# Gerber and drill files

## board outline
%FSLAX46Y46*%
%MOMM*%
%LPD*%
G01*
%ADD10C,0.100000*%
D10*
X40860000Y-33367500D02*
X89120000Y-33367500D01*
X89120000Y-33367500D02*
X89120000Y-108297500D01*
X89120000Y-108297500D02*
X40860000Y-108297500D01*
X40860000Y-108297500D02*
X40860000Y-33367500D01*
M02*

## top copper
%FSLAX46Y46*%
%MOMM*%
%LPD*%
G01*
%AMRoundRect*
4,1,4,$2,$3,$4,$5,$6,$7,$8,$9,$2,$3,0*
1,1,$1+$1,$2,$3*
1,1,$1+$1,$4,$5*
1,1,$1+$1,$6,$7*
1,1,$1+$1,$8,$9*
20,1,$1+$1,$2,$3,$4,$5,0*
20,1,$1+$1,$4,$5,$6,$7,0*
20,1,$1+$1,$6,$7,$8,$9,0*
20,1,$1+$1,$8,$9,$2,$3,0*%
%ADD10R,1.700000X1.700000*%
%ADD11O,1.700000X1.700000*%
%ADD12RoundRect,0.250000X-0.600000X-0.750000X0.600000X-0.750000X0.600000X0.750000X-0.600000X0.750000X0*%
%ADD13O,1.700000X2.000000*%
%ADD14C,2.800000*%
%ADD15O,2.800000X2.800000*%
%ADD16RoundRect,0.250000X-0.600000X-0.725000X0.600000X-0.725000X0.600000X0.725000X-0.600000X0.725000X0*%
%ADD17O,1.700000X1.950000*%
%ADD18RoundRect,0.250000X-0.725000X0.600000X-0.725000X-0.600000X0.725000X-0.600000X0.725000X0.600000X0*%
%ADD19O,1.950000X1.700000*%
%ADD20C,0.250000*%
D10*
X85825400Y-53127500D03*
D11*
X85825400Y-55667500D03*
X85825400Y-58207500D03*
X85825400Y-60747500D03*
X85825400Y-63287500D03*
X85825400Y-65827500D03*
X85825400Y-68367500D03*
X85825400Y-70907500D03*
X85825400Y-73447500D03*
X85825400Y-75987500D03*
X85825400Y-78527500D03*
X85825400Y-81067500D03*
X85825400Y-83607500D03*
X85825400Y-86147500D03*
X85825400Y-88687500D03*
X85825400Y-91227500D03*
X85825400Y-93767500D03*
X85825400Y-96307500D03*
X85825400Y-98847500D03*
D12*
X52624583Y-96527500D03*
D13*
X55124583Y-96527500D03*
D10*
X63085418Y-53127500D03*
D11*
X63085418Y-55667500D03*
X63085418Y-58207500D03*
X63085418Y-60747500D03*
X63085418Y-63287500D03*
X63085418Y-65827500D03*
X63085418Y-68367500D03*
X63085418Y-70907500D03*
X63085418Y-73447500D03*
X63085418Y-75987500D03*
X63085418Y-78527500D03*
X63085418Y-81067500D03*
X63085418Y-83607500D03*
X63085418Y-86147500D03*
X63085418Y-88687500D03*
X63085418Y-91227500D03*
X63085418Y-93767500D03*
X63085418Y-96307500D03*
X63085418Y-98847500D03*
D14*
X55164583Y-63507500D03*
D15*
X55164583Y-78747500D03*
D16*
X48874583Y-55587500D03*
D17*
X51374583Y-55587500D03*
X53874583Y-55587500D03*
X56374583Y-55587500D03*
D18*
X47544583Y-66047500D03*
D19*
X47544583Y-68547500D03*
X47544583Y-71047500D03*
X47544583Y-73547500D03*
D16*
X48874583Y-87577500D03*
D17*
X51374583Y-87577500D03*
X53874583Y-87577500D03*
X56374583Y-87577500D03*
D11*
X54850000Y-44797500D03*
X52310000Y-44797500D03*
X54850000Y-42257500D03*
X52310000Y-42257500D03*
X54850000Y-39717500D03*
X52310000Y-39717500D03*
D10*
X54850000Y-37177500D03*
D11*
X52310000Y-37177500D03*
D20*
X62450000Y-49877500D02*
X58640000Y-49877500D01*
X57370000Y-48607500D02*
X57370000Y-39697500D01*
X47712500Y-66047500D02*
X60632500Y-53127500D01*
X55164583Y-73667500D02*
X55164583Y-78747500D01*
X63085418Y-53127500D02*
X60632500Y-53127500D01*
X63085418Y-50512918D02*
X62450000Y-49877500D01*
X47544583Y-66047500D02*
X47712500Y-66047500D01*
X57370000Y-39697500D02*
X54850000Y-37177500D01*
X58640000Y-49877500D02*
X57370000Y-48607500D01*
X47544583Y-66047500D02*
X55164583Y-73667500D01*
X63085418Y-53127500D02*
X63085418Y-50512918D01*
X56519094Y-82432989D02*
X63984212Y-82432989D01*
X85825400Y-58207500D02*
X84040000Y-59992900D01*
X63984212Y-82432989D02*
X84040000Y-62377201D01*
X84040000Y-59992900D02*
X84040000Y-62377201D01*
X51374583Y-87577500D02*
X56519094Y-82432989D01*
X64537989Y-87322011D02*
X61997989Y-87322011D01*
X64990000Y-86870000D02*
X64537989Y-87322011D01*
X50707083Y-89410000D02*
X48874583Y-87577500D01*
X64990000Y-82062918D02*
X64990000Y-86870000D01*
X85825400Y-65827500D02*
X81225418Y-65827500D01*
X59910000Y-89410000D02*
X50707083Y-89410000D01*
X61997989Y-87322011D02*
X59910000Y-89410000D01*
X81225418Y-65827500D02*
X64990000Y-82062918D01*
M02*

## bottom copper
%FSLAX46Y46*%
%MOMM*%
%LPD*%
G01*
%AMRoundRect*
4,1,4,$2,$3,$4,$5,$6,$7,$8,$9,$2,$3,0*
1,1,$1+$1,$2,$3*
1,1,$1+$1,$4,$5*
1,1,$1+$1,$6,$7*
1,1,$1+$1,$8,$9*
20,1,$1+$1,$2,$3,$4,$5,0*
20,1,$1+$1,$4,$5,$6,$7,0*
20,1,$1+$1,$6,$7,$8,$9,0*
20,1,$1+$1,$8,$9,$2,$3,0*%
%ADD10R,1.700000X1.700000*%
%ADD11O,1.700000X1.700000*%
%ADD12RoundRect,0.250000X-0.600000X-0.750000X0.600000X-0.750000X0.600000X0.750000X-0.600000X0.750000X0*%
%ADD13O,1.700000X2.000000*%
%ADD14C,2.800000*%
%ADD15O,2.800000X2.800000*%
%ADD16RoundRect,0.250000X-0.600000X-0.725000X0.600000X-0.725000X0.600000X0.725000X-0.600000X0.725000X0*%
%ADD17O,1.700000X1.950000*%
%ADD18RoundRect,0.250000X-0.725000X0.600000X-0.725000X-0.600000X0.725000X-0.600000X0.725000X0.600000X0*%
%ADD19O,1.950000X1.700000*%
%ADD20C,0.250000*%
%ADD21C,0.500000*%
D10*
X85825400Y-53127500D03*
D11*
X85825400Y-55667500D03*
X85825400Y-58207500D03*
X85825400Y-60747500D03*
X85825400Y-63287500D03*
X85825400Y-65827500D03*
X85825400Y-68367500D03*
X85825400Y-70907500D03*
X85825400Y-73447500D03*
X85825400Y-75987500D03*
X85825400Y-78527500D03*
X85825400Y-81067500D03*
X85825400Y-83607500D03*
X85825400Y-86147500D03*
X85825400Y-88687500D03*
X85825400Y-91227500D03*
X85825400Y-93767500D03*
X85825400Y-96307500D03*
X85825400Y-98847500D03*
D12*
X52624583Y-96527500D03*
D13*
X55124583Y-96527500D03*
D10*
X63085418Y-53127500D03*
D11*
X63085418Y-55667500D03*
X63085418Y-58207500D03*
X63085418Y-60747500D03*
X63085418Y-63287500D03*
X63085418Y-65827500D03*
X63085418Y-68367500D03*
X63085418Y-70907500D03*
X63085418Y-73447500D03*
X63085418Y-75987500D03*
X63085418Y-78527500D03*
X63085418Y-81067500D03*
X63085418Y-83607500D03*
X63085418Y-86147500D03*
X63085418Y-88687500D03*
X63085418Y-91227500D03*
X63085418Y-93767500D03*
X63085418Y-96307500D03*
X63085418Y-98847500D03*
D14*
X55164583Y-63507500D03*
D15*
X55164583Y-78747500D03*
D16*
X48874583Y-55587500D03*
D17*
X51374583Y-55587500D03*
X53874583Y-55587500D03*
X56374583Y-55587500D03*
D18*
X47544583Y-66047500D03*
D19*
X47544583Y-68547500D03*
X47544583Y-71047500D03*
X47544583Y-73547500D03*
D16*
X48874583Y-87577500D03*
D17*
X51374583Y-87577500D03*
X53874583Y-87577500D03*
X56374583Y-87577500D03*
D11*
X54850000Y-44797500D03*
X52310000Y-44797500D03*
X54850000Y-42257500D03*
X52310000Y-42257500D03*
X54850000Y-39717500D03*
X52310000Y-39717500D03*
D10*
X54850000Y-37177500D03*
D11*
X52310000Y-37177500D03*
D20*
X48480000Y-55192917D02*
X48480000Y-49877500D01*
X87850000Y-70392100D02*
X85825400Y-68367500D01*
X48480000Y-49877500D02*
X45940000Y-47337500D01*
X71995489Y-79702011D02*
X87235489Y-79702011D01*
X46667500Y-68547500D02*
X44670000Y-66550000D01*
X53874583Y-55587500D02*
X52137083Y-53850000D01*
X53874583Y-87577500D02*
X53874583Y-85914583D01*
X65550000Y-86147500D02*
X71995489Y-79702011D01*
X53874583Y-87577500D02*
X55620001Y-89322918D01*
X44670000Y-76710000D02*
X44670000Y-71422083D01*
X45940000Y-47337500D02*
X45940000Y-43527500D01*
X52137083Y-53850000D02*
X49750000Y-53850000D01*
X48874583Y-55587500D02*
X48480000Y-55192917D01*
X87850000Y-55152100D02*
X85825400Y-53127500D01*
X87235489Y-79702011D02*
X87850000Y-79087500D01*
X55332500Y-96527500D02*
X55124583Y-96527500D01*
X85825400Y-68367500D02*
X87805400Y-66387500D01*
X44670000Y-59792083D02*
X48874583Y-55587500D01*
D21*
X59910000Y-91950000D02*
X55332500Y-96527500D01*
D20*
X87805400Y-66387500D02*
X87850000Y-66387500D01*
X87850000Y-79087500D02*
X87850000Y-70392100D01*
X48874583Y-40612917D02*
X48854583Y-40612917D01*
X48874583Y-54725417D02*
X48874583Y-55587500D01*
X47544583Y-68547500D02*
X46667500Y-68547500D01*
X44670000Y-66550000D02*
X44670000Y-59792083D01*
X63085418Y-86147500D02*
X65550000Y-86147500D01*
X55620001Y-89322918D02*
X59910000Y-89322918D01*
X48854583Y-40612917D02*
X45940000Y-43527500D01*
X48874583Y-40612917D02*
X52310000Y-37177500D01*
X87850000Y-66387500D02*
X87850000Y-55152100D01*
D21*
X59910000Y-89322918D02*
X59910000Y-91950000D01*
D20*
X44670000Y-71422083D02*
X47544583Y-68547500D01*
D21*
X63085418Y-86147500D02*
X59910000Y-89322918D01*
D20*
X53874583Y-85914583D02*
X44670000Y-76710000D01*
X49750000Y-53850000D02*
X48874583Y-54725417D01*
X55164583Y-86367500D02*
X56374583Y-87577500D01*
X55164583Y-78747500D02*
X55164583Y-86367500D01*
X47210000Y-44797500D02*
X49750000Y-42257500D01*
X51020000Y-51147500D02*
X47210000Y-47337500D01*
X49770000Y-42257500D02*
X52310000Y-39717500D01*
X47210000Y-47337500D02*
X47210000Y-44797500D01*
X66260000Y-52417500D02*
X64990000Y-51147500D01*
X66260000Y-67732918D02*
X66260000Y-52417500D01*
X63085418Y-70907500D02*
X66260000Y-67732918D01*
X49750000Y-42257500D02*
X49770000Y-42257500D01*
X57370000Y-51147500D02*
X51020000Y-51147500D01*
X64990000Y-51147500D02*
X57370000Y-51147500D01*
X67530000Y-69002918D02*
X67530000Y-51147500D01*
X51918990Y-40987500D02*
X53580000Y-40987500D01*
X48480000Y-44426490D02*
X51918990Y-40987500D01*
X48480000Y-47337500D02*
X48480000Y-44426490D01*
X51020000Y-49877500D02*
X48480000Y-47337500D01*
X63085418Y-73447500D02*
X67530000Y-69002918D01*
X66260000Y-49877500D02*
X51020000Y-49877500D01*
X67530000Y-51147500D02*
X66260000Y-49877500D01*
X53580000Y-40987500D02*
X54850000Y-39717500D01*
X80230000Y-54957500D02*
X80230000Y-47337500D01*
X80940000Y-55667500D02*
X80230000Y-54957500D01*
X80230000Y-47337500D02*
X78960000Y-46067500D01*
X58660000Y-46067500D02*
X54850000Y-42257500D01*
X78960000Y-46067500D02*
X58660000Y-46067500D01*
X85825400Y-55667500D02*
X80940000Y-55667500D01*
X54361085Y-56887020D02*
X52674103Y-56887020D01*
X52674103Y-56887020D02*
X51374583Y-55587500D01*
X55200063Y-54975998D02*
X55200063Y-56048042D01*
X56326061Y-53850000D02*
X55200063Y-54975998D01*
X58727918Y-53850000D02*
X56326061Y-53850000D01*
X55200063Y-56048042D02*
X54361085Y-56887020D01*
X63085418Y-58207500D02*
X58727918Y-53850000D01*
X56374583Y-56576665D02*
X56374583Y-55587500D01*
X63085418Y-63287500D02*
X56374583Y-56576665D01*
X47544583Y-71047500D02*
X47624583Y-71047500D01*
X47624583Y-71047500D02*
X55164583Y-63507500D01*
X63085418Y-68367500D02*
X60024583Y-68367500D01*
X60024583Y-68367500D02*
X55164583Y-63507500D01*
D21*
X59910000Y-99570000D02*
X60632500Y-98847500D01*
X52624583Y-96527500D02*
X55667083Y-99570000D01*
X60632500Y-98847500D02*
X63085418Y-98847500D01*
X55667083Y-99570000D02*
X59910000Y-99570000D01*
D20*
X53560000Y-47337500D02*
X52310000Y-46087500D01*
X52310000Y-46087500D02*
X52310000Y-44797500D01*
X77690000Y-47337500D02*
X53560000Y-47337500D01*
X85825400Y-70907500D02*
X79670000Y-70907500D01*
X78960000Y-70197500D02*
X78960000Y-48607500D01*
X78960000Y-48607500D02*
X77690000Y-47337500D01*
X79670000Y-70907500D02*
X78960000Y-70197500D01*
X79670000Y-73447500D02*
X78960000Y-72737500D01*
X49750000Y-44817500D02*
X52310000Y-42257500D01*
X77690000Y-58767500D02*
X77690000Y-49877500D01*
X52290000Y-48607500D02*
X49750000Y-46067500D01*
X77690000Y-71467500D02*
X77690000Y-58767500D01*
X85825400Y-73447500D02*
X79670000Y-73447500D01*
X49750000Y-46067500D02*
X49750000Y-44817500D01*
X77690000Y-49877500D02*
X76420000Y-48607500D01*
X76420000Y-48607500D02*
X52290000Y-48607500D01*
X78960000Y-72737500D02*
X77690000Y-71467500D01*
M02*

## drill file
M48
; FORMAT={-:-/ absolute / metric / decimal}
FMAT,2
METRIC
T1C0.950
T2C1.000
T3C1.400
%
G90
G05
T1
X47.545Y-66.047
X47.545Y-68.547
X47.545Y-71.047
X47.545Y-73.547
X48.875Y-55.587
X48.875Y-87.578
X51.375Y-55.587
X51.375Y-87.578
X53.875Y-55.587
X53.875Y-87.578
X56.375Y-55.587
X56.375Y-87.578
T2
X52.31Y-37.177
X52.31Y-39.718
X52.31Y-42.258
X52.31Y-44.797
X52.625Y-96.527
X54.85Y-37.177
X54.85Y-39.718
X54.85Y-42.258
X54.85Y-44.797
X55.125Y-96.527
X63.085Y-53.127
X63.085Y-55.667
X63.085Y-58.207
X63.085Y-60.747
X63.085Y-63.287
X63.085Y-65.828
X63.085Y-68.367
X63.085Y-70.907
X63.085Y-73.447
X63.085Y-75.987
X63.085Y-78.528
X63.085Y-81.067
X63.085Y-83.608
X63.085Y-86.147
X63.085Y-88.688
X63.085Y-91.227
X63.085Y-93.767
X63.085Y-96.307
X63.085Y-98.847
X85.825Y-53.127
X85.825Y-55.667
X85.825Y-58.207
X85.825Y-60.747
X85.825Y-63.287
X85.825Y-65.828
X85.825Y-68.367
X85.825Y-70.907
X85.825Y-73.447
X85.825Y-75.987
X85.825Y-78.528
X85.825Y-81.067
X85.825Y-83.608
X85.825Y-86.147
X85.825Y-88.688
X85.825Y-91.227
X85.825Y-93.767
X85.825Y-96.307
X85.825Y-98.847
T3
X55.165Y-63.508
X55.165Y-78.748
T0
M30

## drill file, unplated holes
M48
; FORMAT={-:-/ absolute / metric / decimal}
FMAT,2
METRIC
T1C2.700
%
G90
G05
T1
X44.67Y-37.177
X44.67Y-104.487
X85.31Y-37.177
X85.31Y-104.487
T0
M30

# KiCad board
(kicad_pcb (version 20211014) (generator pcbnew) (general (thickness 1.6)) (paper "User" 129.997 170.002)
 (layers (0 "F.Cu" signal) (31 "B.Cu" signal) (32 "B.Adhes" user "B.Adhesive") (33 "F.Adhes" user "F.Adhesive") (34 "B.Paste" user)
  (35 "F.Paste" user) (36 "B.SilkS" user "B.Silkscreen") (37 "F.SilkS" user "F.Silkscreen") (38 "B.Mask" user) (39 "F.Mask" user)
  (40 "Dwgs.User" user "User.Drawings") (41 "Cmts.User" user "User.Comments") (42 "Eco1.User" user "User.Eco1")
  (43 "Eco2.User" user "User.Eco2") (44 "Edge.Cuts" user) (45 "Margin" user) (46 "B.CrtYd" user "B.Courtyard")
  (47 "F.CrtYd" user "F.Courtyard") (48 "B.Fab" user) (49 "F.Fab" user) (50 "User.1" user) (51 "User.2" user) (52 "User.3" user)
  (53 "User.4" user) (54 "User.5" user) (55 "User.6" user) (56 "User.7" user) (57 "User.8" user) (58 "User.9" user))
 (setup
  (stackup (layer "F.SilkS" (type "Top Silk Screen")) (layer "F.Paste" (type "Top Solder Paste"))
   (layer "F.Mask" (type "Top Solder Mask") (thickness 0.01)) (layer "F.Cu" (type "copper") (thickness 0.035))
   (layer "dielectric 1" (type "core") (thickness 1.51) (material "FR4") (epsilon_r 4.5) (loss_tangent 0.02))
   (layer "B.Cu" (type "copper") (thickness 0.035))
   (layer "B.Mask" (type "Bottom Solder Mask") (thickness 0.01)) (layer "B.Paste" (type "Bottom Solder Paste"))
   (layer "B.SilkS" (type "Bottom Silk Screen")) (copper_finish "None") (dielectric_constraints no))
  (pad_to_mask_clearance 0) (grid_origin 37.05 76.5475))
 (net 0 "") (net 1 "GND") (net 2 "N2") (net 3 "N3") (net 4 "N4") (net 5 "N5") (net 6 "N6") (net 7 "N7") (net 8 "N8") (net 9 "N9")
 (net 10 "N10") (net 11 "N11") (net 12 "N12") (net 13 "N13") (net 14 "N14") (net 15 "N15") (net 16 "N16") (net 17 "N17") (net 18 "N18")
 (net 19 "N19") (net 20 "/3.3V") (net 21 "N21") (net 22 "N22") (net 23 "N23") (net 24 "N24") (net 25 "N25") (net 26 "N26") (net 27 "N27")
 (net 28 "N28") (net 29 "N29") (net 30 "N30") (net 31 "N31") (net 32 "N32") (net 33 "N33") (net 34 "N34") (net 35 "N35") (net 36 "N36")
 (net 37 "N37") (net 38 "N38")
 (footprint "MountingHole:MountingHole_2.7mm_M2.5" (layer "F.Cu") (at 44.67 37.1775)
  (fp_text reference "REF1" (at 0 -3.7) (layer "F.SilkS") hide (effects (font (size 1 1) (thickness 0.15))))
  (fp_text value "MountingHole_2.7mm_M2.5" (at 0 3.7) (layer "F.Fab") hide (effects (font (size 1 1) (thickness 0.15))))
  (pad "" np_thru_hole circle (at 0 0) (size 2.7 2.7) (drill 2.7) (layers *.Cu *.Mask)))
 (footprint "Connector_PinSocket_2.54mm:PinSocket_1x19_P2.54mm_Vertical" (layer "F.Cu") (at 85.8254 53.1275)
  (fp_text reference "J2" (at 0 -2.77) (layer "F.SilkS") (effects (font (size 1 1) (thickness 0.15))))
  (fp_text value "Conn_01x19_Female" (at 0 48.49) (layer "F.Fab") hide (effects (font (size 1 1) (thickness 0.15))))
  (pad "1" thru_hole rect (at 0 0) (size 1.7 1.7) (drill 1) (layers *.Cu *.Mask) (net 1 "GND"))
  (pad "2" thru_hole oval (at 0 2.54) (size 1.7 1.7) (drill 1) (layers *.Cu *.Mask) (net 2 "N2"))
  (pad "3" thru_hole oval (at 0 5.08) (size 1.7 1.7) (drill 1) (layers *.Cu *.Mask) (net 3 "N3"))
  (pad "4" thru_hole oval (at 0 7.62) (size 1.7 1.7) (drill 1) (layers *.Cu *.Mask) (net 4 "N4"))
  (pad "5" thru_hole oval (at 0 10.16) (size 1.7 1.7) (drill 1) (layers *.Cu *.Mask) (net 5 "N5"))
  (pad "6" thru_hole oval (at 0 12.7) (size 1.7 1.7) (drill 1) (layers *.Cu *.Mask) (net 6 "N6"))
  (pad "7" thru_hole oval (at 0 15.24) (size 1.7 1.7) (drill 1) (layers *.Cu *.Mask) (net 1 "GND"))
  (pad "8" thru_hole oval (at 0 17.78) (size 1.7 1.7) (drill 1) (layers *.Cu *.Mask) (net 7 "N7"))
  (pad "9" thru_hole oval (at 0 20.32) (size 1.7 1.7) (drill 1) (layers *.Cu *.Mask) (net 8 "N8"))
  (pad "10" thru_hole oval (at 0 22.86) (size 1.7 1.7) (drill 1) (layers *.Cu *.Mask) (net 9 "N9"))
  (pad "11" thru_hole oval (at 0 25.4) (size 1.7 1.7) (drill 1) (layers *.Cu *.Mask) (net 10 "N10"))
  (pad "12" thru_hole oval (at 0 27.94) (size 1.7 1.7) (drill 1) (layers *.Cu *.Mask) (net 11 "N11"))
  (pad "13" thru_hole oval (at 0 30.48) (size 1.7 1.7) (drill 1) (layers *.Cu *.Mask) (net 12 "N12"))
  (pad "14" thru_hole oval (at 0 33.02) (size 1.7 1.7) (drill 1) (layers *.Cu *.Mask) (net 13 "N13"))
  (pad "15" thru_hole oval (at 0 35.56) (size 1.7 1.7) (drill 1) (layers *.Cu *.Mask) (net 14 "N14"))
  (pad "16" thru_hole oval (at 0 38.1) (size 1.7 1.7) (drill 1) (layers *.Cu *.Mask) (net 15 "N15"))
  (pad "17" thru_hole oval (at 0 40.64) (size 1.7 1.7) (drill 1) (layers *.Cu *.Mask) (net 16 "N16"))
  (pad "18" thru_hole oval (at 0 43.18) (size 1.7 1.7) (drill 1) (layers *.Cu *.Mask) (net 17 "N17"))
  (pad "19" thru_hole oval (at 0 45.72) (size 1.7 1.7) (drill 1) (layers *.Cu *.Mask) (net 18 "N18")))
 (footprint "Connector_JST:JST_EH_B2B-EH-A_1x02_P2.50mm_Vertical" (layer "F.Cu") (at 52.624583 96.5275)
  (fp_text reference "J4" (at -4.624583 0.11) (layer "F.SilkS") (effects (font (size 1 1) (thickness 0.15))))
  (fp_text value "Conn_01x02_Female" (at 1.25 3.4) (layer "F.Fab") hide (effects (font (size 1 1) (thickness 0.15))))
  (pad "1" thru_hole roundrect (at 0 0) (size 1.7 2) (drill 1) (layers *.Cu *.Mask) (roundrect_rratio 0.1470588235) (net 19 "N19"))
  (pad "2" thru_hole oval (at 2.5 0) (size 1.7 2) (drill 1) (layers *.Cu *.Mask) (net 1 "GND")))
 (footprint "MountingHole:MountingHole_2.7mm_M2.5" (layer "F.Cu") (at 85.31 104.4875)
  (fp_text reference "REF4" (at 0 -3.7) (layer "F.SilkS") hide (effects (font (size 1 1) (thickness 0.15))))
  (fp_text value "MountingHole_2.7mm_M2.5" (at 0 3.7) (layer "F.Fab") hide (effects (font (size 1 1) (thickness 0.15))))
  (pad "" np_thru_hole circle (at 0 0) (size 2.7 2.7) (drill 2.7) (layers *.Cu *.Mask)))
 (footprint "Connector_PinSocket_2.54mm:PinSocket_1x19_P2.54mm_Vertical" (layer "F.Cu") (at 63.085418 53.1275)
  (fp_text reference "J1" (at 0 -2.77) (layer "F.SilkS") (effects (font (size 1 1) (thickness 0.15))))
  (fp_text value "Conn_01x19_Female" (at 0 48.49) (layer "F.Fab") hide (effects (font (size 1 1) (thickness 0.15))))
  (pad "1" thru_hole rect (at 0 0) (size 1.7 1.7) (drill 1) (layers *.Cu *.Mask) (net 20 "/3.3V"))
  (pad "2" thru_hole oval (at 0 2.54) (size 1.7 1.7) (drill 1) (layers *.Cu *.Mask) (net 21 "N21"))
  (pad "3" thru_hole oval (at 0 5.08) (size 1.7 1.7) (drill 1) (layers *.Cu *.Mask) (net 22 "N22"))
  (pad "4" thru_hole oval (at 0 7.62) (size 1.7 1.7) (drill 1) (layers *.Cu *.Mask) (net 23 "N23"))
  (pad "5" thru_hole oval (at 0 10.16) (size 1.7 1.7) (drill 1) (layers *.Cu *.Mask) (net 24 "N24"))
  (pad "6" thru_hole oval (at 0 12.7) (size 1.7 1.7) (drill 1) (layers *.Cu *.Mask) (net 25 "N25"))
  (pad "7" thru_hole oval (at 0 15.24) (size 1.7 1.7) (drill 1) (layers *.Cu *.Mask) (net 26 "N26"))
  (pad "8" thru_hole oval (at 0 17.78) (size 1.7 1.7) (drill 1) (layers *.Cu *.Mask) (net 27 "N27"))
  (pad "9" thru_hole oval (at 0 20.32) (size 1.7 1.7) (drill 1) (layers *.Cu *.Mask) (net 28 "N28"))
  (pad "10" thru_hole oval (at 0 22.86) (size 1.7 1.7) (drill 1) (layers *.Cu *.Mask) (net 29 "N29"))
  (pad "11" thru_hole oval (at 0 25.4) (size 1.7 1.7) (drill 1) (layers *.Cu *.Mask) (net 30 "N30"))
  (pad "12" thru_hole oval (at 0 27.94) (size 1.7 1.7) (drill 1) (layers *.Cu *.Mask) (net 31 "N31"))
  (pad "13" thru_hole oval (at 0 30.48) (size 1.7 1.7) (drill 1) (layers *.Cu *.Mask) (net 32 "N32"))
  (pad "14" thru_hole oval (at 0 33.02) (size 1.7 1.7) (drill 1) (layers *.Cu *.Mask) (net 1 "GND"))
  (pad "15" thru_hole oval (at 0 35.56) (size 1.7 1.7) (drill 1) (layers *.Cu *.Mask) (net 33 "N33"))
  (pad "16" thru_hole oval (at 0 38.1) (size 1.7 1.7) (drill 1) (layers *.Cu *.Mask) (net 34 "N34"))
  (pad "17" thru_hole oval (at 0 40.64) (size 1.7 1.7) (drill 1) (layers *.Cu *.Mask) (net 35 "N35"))
  (pad "18" thru_hole oval (at 0 43.18) (size 1.7 1.7) (drill 1) (layers *.Cu *.Mask) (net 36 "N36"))
  (pad "19" thru_hole oval (at 0 45.72) (size 1.7 1.7) (drill 1) (layers *.Cu *.Mask) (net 19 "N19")))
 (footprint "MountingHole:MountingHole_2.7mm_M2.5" (layer "F.Cu") (at 44.67 104.4875)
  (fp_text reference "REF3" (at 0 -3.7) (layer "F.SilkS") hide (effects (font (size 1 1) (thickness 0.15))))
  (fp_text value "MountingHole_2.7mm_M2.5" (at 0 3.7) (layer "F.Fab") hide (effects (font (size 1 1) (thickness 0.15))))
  (pad "" np_thru_hole circle (at 0 0) (size 2.7 2.7) (drill 2.7) (layers *.Cu *.Mask)))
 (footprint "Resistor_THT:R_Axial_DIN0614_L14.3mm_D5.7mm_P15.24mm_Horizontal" (layer "F.Cu") (at 55.164583 63.5075 -90)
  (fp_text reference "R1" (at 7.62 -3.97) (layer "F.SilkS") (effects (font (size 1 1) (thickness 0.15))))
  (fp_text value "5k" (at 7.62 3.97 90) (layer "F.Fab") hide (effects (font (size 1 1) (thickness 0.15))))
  (pad "1" thru_hole circle (at 0 0 270) (size 2.8 2.8) (drill 1.4) (layers *.Cu *.Mask) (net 26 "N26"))
  (pad "2" thru_hole oval (at 15.24 0 270) (size 2.8 2.8) (drill 1.4) (layers *.Cu *.Mask) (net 20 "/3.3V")))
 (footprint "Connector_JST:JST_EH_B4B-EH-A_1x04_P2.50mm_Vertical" (layer "F.Cu") (at 48.874583 55.5875)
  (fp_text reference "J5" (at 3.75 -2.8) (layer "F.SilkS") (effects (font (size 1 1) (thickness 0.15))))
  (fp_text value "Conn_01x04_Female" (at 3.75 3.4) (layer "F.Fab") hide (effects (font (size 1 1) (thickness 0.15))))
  (pad "1" thru_hole roundrect (at 0 0) (size 1.7 1.95) (drill 0.95) (layers *.Cu *.Mask) (roundrect_rratio 0.1470588235) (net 1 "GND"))
  (pad "2" thru_hole oval (at 2.5 0) (size 1.7 1.95) (drill 0.95) (layers *.Cu *.Mask) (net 22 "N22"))
  (pad "3" thru_hole oval (at 5 0) (size 1.7 1.95) (drill 0.95) (layers *.Cu *.Mask) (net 1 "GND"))
  (pad "4" thru_hole oval (at 7.5 0) (size 1.7 1.95) (drill 0.95) (layers *.Cu *.Mask) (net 24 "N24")))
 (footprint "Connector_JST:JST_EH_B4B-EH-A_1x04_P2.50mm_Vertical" (layer "F.Cu") (at 47.544583 66.0475 -90)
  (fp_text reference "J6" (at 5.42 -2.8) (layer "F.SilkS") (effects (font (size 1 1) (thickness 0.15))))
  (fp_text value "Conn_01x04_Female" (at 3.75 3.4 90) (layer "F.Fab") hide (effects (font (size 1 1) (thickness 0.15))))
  (pad "1" thru_hole roundrect (at 0 0 270) (size 1.7 1.95) (drill 0.95) (layers *.Cu *.Mask) (roundrect_rratio 0.1470588235)
   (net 20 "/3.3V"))
  (pad "2" thru_hole oval (at 2.5 0 270) (size 1.7 1.95) (drill 0.95) (layers *.Cu *.Mask) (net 1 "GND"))
  (pad "3" thru_hole oval (at 5 0 270) (size 1.7 1.95) (drill 0.95) (layers *.Cu *.Mask) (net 26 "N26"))
  (pad "4" thru_hole oval (at 7.5 0 270) (size 1.7 1.95) (drill 0.95) (layers *.Cu *.Mask) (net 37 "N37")))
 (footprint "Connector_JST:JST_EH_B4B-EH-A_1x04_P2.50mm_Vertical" (layer "F.Cu") (at 48.874583 87.5775)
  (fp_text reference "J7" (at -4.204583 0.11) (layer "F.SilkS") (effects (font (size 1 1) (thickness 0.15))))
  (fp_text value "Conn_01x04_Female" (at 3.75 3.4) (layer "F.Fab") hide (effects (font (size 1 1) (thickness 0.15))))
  (pad "1" thru_hole roundrect (at 0 0) (size 1.7 1.95) (drill 0.95) (layers *.Cu *.Mask) (roundrect_rratio 0.1470588235) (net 6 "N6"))
  (pad "2" thru_hole oval (at 2.5 0) (size 1.7 1.95) (drill 0.95) (layers *.Cu *.Mask) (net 3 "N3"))
  (pad "3" thru_hole oval (at 5 0) (size 1.7 1.95) (drill 0.95) (layers *.Cu *.Mask) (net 1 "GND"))
  (pad "4" thru_hole oval (at 7.5 0) (size 1.7 1.95) (drill 0.95) (layers *.Cu *.Mask) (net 20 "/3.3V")))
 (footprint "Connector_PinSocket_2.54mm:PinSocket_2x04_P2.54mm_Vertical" (layer "F.Cu") (at 54.85 37.1775)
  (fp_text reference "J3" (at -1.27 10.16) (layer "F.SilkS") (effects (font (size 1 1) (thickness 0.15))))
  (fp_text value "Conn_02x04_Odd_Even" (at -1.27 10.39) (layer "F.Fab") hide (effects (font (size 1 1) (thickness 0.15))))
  (pad "1" thru_hole oval (at 0 7.62) (size 1.7 1.7) (drill 1) (layers *.Cu *.Mask) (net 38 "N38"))
  (pad "2" thru_hole oval (at -2.54 7.62) (size 1.7 1.7) (drill 1) (layers *.Cu *.Mask) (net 7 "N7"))
  (pad "3" thru_hole oval (at 0 5.08) (size 1.7 1.7) (drill 1) (layers *.Cu *.Mask) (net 2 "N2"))
  (pad "4" thru_hole oval (at -2.54 5.08) (size 1.7 1.7) (drill 1) (layers *.Cu *.Mask) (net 8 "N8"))
  (pad "5" thru_hole oval (at 0 2.54) (size 1.7 1.7) (drill 1) (layers *.Cu *.Mask) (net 28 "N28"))
  (pad "6" thru_hole oval (at -2.54 2.54) (size 1.7 1.7) (drill 1) (layers *.Cu *.Mask) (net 27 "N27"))
  (pad "7" thru_hole rect (at 0 0) (size 1.7 1.7) (drill 1) (layers *.Cu *.Mask) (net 20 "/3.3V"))
  (pad "8" thru_hole oval (at -2.54 0) (size 1.7 1.7) (drill 1) (layers *.Cu *.Mask) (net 1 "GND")))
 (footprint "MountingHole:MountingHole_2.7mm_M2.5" (layer "F.Cu") (at 85.31 37.1775)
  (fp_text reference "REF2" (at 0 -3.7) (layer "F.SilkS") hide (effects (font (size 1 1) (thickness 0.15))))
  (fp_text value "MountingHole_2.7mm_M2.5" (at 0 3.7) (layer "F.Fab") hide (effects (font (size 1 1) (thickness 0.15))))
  (pad "" np_thru_hole circle (at 0 0) (size 2.7 2.7) (drill 2.7) (layers *.Cu *.Mask)))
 (gr_rect (start 40.86 33.3675) (end 89.12 108.2975) (layer "Edge.Cuts") (width 0.1) (fill none))
 (segment (start 48.48 55.192917) (end 48.48 49.8775) (width 0.25) (layer "B.Cu") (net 1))
 (segment (start 87.85 70.3921) (end 85.8254 68.3675) (width 0.25) (layer "B.Cu") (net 1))
 (segment (start 48.48 49.8775) (end 45.94 47.3375) (width 0.25) (layer "B.Cu") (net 1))
 (segment (start 71.995489 79.702011) (end 87.235489 79.702011) (width 0.25) (layer "B.Cu") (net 1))
 (segment (start 46.6675 68.5475) (end 44.67 66.55) (width 0.25) (layer "B.Cu") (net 1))
 (segment (start 53.874583 55.5875) (end 52.137083 53.85) (width 0.25) (layer "B.Cu") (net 1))
 (segment (start 53.874583 87.5775) (end 53.874583 85.914583) (width 0.25) (layer "B.Cu") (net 1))
 (segment (start 65.55 86.1475) (end 71.995489 79.702011) (width 0.25) (layer "B.Cu") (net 1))
 (segment (start 53.874583 87.5775) (end 55.620001 89.322918) (width 0.25) (layer "B.Cu") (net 1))
 (segment (start 44.67 76.71) (end 44.67 71.422083) (width 0.25) (layer "B.Cu") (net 1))
 (segment (start 45.94 47.3375) (end 45.94 43.5275) (width 0.25) (layer "B.Cu") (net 1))
 (segment (start 52.137083 53.85) (end 49.75 53.85) (width 0.25) (layer "B.Cu") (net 1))
 (segment (start 48.874583 55.5875) (end 48.48 55.192917) (width 0.25) (layer "B.Cu") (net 1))
 (segment (start 87.85 55.1521) (end 85.8254 53.1275) (width 0.25) (layer "B.Cu") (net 1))
 (segment (start 87.235489 79.702011) (end 87.85 79.0875) (width 0.25) (layer "B.Cu") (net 1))
 (segment (start 55.3325 96.5275) (end 55.124583 96.5275) (width 0.25) (layer "B.Cu") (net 1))
 (segment (start 85.8254 68.3675) (end 87.8054 66.3875) (width 0.25) (layer "B.Cu") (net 1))
 (segment (start 44.67 59.792083) (end 48.874583 55.5875) (width 0.25) (layer "B.Cu") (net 1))
 (segment (start 59.91 91.95) (end 55.3325 96.5275) (width 0.5) (layer "B.Cu") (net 1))
 (segment (start 87.8054 66.3875) (end 87.85 66.3875) (width 0.25) (layer "B.Cu") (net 1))
 (segment (start 87.85 79.0875) (end 87.85 70.3921) (width 0.25) (layer "B.Cu") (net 1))
 (segment (start 48.874583 40.612917) (end 48.854583 40.612917) (width 0.25) (layer "B.Cu") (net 1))
 (segment (start 48.874583 54.725417) (end 48.874583 55.5875) (width 0.25) (layer "B.Cu") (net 1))
 (segment (start 47.544583 68.5475) (end 46.6675 68.5475) (width 0.25) (layer "B.Cu") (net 1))
 (segment (start 44.67 66.55) (end 44.67 59.792083) (width 0.25) (layer "B.Cu") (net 1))
 (segment (start 63.085418 86.1475) (end 65.55 86.1475) (width 0.25) (layer "B.Cu") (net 1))
 (segment (start 55.620001 89.322918) (end 59.91 89.322918) (width 0.25) (layer "B.Cu") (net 1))
 (segment (start 48.854583 40.612917) (end 45.94 43.5275) (width 0.25) (layer "B.Cu") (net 1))
 (segment (start 48.874583 40.612917) (end 52.31 37.1775) (width 0.25) (layer "B.Cu") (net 1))
 (segment (start 87.85 66.3875) (end 87.85 55.1521) (width 0.25) (layer "B.Cu") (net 1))
 (segment (start 59.91 89.322918) (end 59.91 91.95) (width 0.5) (layer "B.Cu") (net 1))
 (segment (start 44.67 71.422083) (end 47.544583 68.5475) (width 0.25) (layer "B.Cu") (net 1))
 (segment (start 63.085418 86.1475) (end 59.91 89.322918) (width 0.5) (layer "B.Cu") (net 1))
 (segment (start 53.874583 85.914583) (end 44.67 76.71) (width 0.25) (layer "B.Cu") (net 1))
 (segment (start 49.75 53.85) (end 48.874583 54.725417) (width 0.25) (layer "B.Cu") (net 1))
 (segment (start 62.45 49.8775) (end 58.64 49.8775) (width 0.25) (layer "F.Cu") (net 20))
 (segment (start 57.37 48.6075) (end 57.37 39.6975) (width 0.25) (layer "F.Cu") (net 20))
 (segment (start 47.7125 66.0475) (end 60.6325 53.1275) (width 0.25) (layer "F.Cu") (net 20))
 (segment (start 55.164583 73.6675) (end 55.164583 78.7475) (width 0.25) (layer "F.Cu") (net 20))
 (segment (start 63.085418 53.1275) (end 60.6325 53.1275) (width 0.25) (layer "F.Cu") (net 20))
 (segment (start 63.085418 50.512918) (end 62.45 49.8775) (width 0.25) (layer "F.Cu") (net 20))
 (segment (start 47.544583 66.0475) (end 47.7125 66.0475) (width 0.25) (layer "F.Cu") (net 20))
 (segment (start 57.37 39.6975) (end 54.85 37.1775) (width 0.25) (layer "F.Cu") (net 20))
 (segment (start 58.64 49.8775) (end 57.37 48.6075) (width 0.25) (layer "F.Cu") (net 20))
 (segment (start 47.544583 66.0475) (end 55.164583 73.6675) (width 0.25) (layer "F.Cu") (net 20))
 (segment (start 63.085418 53.1275) (end 63.085418 50.512918) (width 0.25) (layer "F.Cu") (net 20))
 (segment (start 55.164583 86.3675) (end 56.374583 87.5775) (width 0.25) (layer "B.Cu") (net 20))
 (segment (start 55.164583 78.7475) (end 55.164583 86.3675) (width 0.25) (layer "B.Cu") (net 20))
 (segment (start 47.21 44.7975) (end 49.75 42.2575) (width 0.25) (layer "B.Cu") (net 27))
 (segment (start 51.02 51.1475) (end 47.21 47.3375) (width 0.25) (layer "B.Cu") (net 27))
 (segment (start 49.77 42.2575) (end 52.31 39.7175) (width 0.25) (layer "B.Cu") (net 27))
 (segment (start 47.21 47.3375) (end 47.21 44.7975) (width 0.25) (layer "B.Cu") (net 27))
 (segment (start 66.26 52.4175) (end 64.99 51.1475) (width 0.25) (layer "B.Cu") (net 27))
 (segment (start 66.26 67.732918) (end 66.26 52.4175) (width 0.25) (layer "B.Cu") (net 27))
 (segment (start 63.085418 70.9075) (end 66.26 67.732918) (width 0.25) (layer "B.Cu") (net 27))
 (segment (start 49.75 42.2575) (end 49.77 42.2575) (width 0.25) (layer "B.Cu") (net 27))
 (segment (start 57.37 51.1475) (end 51.02 51.1475) (width 0.25) (layer "B.Cu") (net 27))
 (segment (start 64.99 51.1475) (end 57.37 51.1475) (width 0.25) (layer "B.Cu") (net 27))
 (segment (start 67.53 69.002918) (end 67.53 51.1475) (width 0.25) (layer "B.Cu") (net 28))
 (segment (start 51.91899 40.9875) (end 53.58 40.9875) (width 0.25) (layer "B.Cu") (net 28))
 (segment (start 48.48 44.42649) (end 51.91899 40.9875) (width 0.25) (layer "B.Cu") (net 28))
 (segment (start 48.48 47.3375) (end 48.48 44.42649) (width 0.25) (layer "B.Cu") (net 28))
 (segment (start 51.02 49.8775) (end 48.48 47.3375) (width 0.25) (layer "B.Cu") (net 28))
 (segment (start 63.085418 73.4475) (end 67.53 69.002918) (width 0.25) (layer "B.Cu") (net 28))
 (segment (start 66.26 49.8775) (end 51.02 49.8775) (width 0.25) (layer "B.Cu") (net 28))
 (segment (start 67.53 51.1475) (end 66.26 49.8775) (width 0.25) (layer "B.Cu") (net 28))
 (segment (start 53.58 40.9875) (end 54.85 39.7175) (width 0.25) (layer "B.Cu") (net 28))
 (segment (start 80.23 54.9575) (end 80.23 47.3375) (width 0.25) (layer "B.Cu") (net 2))
 (segment (start 80.94 55.6675) (end 80.23 54.9575) (width 0.25) (layer "B.Cu") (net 2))
 (segment (start 80.23 47.3375) (end 78.96 46.0675) (width 0.25) (layer "B.Cu") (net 2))
 (segment (start 58.66 46.0675) (end 54.85 42.2575) (width 0.25) (layer "B.Cu") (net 2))
 (segment (start 78.96 46.0675) (end 58.66 46.0675) (width 0.25) (layer "B.Cu") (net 2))
 (segment (start 85.8254 55.6675) (end 80.94 55.6675) (width 0.25) (layer "B.Cu") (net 2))
 (segment (start 54.361085 56.88702) (end 52.674103 56.88702) (width 0.25) (layer "B.Cu") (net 22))
 (segment (start 52.674103 56.88702) (end 51.374583 55.5875) (width 0.25) (layer "B.Cu") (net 22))
 (segment (start 55.200063 54.975998) (end 55.200063 56.048042) (width 0.25) (layer "B.Cu") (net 22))
 (segment (start 56.326061 53.85) (end 55.200063 54.975998) (width 0.25) (layer "B.Cu") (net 22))
 (segment (start 58.727918 53.85) (end 56.326061 53.85) (width 0.25) (layer "B.Cu") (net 22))
 (segment (start 55.200063 56.048042) (end 54.361085 56.88702) (width 0.25) (layer "B.Cu") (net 22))
 (segment (start 63.085418 58.2075) (end 58.727918 53.85) (width 0.25) (layer "B.Cu") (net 22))
 (segment (start 56.374583 56.576665) (end 56.374583 55.5875) (width 0.25) (layer "B.Cu") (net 24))
 (segment (start 63.085418 63.2875) (end 56.374583 56.576665) (width 0.25) (layer "B.Cu") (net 24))
 (segment (start 47.544583 71.0475) (end 47.624583 71.0475) (width 0.25) (layer "B.Cu") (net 26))
 (segment (start 47.624583 71.0475) (end 55.164583 63.5075) (width 0.25) (layer "B.Cu") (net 26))
 (segment (start 63.085418 68.3675) (end 60.024583 68.3675) (width 0.25) (layer "B.Cu") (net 26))
 (segment (start 60.024583 68.3675) (end 55.164583 63.5075) (width 0.25) (layer "B.Cu") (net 26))
 (segment (start 59.91 99.57) (end 60.6325 98.8475) (width 0.5) (layer "B.Cu") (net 19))
 (segment (start 52.624583 96.5275) (end 55.667083 99.57) (width 0.5) (layer "B.Cu") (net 19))
 (segment (start 60.6325 98.8475) (end 63.085418 98.8475) (width 0.5) (layer "B.Cu") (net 19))
 (segment (start 55.667083 99.57) (end 59.91 99.57) (width 0.5) (layer "B.Cu") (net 19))
 (segment (start 56.519094 82.432989) (end 63.984212 82.432989) (width 0.25) (layer "F.Cu") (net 3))
 (segment (start 85.8254 58.2075) (end 84.04 59.9929) (width 0.25) (layer "F.Cu") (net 3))
 (segment (start 63.984212 82.432989) (end 84.04 62.377201) (width 0.25) (layer "F.Cu") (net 3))
 (segment (start 84.04 59.9929) (end 84.04 62.377201) (width 0.25) (layer "F.Cu") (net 3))
 (segment (start 51.374583 87.5775) (end 56.519094 82.432989) (width 0.25) (layer "F.Cu") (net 3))
 (segment (start 64.537989 87.322011) (end 61.997989 87.322011) (width 0.25) (layer "F.Cu") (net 6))
 (segment (start 64.99 86.87) (end 64.537989 87.322011) (width 0.25) (layer "F.Cu") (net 6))
 (segment (start 50.707083 89.41) (end 48.874583 87.5775) (width 0.25) (layer "F.Cu") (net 6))
 (segment (start 64.99 82.062918) (end 64.99 86.87) (width 0.25) (layer "F.Cu") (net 6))
 (segment (start 85.8254 65.8275) (end 81.225418 65.8275) (width 0.25) (layer "F.Cu") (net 6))
 (segment (start 59.91 89.41) (end 50.707083 89.41) (width 0.25) (layer "F.Cu") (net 6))
 (segment (start 61.997989 87.322011) (end 59.91 89.41) (width 0.25) (layer "F.Cu") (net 6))
 (segment (start 81.225418 65.8275) (end 64.99 82.062918) (width 0.25) (layer "F.Cu") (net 6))
 (segment (start 53.56 47.3375) (end 52.31 46.0875) (width 0.25) (layer "B.Cu") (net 7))
 (segment (start 52.31 46.0875) (end 52.31 44.7975) (width 0.25) (layer "B.Cu") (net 7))
 (segment (start 77.69 47.3375) (end 53.56 47.3375) (width 0.25) (layer "B.Cu") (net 7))
 (segment (start 85.8254 70.9075) (end 79.67 70.9075) (width 0.25) (layer "B.Cu") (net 7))
 (segment (start 78.96 70.1975) (end 78.96 48.6075) (width 0.25) (layer "B.Cu") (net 7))
 (segment (start 78.96 48.6075) (end 77.69 47.3375) (width 0.25) (layer "B.Cu") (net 7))
 (segment (start 79.67 70.9075) (end 78.96 70.1975) (width 0.25) (layer "B.Cu") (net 7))
 (segment (start 79.67 73.4475) (end 78.96 72.7375) (width 0.25) (layer "B.Cu") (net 8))
 (segment (start 49.75 44.8175) (end 52.31 42.2575) (width 0.25) (layer "B.Cu") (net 8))
 (segment (start 77.69 58.7675) (end 77.69 49.8775) (width 0.25) (layer "B.Cu") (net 8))
 (segment (start 52.29 48.6075) (end 49.75 46.0675) (width 0.25) (layer "B.Cu") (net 8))
 (segment (start 77.69 71.4675) (end 77.69 58.7675) (width 0.25) (layer "B.Cu") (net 8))
 (segment (start 85.8254 73.4475) (end 79.67 73.4475) (width 0.25) (layer "B.Cu") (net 8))
 (segment (start 49.75 46.0675) (end 49.75 44.8175) (width 0.25) (layer "B.Cu") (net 8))
 (segment (start 77.69 49.8775) (end 76.42 48.6075) (width 0.25) (layer "B.Cu") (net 8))
 (segment (start 76.42 48.6075) (end 52.29 48.6075) (width 0.25) (layer "B.Cu") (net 8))
 (segment (start 78.96 72.7375) (end 77.69 71.4675) (width 0.25) (layer "B.Cu") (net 8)))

